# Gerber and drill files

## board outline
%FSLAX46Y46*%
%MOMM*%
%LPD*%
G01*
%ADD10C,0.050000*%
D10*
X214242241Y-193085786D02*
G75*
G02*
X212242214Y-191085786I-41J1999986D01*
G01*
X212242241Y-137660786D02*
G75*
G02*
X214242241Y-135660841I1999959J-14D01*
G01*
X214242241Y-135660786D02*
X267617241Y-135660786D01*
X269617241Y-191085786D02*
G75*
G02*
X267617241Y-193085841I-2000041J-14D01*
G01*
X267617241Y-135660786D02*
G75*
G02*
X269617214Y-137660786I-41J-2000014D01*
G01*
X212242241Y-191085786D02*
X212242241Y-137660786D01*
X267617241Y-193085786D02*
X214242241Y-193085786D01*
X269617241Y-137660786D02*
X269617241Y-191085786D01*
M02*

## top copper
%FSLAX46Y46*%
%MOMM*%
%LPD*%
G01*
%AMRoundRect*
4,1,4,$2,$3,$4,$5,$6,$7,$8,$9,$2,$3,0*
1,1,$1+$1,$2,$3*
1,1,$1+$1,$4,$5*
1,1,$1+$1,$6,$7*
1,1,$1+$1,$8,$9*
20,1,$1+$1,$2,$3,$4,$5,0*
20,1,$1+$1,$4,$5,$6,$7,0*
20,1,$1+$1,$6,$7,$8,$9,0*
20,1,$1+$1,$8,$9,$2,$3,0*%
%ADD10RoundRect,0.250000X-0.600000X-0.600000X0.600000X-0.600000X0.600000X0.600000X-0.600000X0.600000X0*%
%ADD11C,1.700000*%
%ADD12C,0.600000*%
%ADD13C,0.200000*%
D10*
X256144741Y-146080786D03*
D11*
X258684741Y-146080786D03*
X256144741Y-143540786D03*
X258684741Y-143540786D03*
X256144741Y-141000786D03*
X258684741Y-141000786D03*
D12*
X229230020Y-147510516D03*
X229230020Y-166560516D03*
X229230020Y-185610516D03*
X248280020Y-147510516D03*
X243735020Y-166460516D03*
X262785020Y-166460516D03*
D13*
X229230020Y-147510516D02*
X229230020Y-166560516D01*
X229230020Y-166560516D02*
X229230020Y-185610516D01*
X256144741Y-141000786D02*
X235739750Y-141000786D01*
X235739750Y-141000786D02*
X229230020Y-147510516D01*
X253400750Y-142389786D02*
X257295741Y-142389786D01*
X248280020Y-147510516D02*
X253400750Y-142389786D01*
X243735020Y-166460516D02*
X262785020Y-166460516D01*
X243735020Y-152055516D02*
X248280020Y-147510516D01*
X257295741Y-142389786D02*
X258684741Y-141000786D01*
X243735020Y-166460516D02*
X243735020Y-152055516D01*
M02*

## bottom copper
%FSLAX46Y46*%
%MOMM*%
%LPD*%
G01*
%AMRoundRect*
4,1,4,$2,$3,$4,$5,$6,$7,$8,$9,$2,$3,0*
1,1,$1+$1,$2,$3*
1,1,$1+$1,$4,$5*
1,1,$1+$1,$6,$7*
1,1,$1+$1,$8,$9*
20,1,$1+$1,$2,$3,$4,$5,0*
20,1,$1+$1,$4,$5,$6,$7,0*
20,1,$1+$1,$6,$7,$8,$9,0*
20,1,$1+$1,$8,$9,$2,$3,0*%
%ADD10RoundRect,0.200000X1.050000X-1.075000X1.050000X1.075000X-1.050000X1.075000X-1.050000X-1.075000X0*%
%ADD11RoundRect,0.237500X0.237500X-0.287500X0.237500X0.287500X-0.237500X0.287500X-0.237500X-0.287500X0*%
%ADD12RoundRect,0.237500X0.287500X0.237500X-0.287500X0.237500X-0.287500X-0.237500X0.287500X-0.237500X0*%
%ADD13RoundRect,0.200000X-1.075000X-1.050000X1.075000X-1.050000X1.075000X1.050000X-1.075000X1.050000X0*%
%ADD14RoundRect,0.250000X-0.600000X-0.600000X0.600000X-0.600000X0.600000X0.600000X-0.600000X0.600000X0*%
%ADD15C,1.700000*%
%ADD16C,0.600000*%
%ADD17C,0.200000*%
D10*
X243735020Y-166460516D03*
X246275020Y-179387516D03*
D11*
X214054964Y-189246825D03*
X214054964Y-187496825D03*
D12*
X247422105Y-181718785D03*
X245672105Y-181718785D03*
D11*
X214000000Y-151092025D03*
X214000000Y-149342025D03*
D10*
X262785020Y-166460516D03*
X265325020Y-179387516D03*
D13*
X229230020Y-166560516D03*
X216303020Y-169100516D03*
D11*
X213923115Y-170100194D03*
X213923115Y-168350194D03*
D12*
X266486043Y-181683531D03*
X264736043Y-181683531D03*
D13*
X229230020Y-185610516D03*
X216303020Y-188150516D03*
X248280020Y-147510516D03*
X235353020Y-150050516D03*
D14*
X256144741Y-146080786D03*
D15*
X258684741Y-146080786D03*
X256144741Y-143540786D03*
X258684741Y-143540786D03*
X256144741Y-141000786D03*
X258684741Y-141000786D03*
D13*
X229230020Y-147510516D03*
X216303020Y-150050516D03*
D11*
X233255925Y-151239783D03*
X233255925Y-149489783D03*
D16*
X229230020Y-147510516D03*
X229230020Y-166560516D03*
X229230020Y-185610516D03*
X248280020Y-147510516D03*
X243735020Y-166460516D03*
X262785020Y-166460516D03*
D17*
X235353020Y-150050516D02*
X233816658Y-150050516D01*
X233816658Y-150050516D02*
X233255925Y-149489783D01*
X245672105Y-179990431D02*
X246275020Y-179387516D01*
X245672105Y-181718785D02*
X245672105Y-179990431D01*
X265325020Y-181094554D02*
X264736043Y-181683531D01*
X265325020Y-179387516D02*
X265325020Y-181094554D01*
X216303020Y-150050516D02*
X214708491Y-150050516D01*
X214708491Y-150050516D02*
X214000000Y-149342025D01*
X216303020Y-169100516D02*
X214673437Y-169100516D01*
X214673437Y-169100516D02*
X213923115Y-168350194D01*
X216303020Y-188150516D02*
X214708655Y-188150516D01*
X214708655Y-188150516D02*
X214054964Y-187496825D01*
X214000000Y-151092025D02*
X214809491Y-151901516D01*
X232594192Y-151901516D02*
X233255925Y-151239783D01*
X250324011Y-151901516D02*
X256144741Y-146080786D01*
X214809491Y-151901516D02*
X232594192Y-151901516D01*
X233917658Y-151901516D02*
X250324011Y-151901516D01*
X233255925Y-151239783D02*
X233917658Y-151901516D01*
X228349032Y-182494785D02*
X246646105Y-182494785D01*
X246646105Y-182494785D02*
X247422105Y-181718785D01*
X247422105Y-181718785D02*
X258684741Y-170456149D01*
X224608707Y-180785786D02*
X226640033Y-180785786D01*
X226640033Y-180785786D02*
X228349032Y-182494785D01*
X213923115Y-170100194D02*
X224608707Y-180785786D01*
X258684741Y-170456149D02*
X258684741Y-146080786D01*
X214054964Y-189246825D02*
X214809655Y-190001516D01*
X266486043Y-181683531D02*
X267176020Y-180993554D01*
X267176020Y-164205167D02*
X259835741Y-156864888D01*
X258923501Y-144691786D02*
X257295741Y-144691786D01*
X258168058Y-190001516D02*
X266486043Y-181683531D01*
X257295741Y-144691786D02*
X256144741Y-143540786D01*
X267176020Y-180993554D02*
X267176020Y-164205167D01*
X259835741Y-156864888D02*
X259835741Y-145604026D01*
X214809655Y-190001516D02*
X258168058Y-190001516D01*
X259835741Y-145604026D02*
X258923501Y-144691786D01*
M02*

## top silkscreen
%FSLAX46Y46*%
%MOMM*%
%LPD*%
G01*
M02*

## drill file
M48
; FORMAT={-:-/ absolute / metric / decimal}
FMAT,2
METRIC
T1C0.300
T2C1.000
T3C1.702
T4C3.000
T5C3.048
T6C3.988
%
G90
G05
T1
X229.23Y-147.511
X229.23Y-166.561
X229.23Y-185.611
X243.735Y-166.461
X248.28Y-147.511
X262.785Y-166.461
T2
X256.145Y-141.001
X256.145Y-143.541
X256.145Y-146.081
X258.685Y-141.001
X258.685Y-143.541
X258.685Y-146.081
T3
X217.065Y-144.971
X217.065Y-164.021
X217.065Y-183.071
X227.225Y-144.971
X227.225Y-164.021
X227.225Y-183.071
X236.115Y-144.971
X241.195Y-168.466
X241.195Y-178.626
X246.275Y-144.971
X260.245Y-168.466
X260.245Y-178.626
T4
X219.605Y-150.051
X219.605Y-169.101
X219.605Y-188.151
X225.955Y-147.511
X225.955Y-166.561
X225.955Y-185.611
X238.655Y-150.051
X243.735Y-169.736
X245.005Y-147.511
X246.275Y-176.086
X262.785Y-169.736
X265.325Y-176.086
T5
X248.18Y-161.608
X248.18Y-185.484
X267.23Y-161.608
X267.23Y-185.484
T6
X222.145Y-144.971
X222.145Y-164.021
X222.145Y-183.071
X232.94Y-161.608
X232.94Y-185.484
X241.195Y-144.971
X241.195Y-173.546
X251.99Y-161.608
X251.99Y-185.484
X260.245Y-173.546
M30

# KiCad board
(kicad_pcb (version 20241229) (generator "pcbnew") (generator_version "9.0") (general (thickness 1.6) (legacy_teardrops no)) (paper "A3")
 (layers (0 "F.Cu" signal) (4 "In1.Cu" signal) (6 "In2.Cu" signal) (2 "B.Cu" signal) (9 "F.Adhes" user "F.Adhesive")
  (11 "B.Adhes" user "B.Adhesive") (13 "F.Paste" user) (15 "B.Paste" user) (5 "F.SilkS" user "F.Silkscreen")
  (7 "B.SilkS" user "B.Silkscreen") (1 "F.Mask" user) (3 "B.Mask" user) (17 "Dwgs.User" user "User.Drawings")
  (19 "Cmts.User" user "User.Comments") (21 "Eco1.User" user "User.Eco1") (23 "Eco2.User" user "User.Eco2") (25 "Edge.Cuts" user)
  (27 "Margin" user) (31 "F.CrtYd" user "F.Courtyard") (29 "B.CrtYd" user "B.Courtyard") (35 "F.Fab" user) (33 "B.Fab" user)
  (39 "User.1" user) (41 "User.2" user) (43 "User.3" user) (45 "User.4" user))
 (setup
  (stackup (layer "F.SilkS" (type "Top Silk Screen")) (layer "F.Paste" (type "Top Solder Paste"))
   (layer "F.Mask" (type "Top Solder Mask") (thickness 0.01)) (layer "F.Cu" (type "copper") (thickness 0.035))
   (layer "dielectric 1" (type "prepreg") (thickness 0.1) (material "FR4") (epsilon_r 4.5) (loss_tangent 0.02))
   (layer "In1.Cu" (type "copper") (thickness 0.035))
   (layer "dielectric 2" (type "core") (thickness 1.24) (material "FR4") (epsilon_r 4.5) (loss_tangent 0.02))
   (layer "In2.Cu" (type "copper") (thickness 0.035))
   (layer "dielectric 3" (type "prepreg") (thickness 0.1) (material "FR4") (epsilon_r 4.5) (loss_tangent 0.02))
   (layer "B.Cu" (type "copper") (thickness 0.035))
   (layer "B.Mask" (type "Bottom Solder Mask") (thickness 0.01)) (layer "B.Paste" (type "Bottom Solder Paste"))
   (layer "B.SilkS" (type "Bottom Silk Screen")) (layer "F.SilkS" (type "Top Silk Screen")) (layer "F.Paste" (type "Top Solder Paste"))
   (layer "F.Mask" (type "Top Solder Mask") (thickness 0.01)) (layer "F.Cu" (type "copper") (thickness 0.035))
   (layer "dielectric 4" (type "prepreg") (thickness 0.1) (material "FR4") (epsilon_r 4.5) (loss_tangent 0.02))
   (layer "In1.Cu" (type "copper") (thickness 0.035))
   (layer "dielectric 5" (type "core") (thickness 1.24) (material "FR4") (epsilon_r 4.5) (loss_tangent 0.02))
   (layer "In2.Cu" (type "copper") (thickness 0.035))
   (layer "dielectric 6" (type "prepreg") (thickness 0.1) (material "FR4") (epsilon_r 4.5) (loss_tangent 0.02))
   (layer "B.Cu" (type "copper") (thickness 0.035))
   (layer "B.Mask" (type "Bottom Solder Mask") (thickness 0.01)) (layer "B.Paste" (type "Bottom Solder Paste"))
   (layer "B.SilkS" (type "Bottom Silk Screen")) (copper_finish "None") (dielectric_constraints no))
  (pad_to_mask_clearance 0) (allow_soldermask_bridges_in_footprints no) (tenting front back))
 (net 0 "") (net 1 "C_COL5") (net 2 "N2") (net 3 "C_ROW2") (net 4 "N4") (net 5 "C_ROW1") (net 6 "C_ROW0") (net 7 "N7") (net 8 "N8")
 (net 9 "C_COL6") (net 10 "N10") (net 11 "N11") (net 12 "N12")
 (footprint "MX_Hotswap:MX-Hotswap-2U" (layer "B.Cu") (at 241.19502 173.545516 90)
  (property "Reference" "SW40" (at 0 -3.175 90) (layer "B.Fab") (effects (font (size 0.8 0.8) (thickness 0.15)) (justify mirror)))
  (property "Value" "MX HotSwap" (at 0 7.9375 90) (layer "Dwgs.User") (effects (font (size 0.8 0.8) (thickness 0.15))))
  (pad "" np_thru_hole circle (at -11.938 -8.255 90) (size 3.9878 3.9878) (drill 3.9878) (layers "*.Cu" "*.Mask"))
  (pad "" np_thru_hole circle (at -11.938 6.985 90) (size 3.048 3.048) (drill 3.048) (layers "*.Cu" "*.Mask"))
  (pad "" np_thru_hole circle (at -5.08 0 138.099) (size 1.7018 1.7018) (drill 1.7018) (layers "*.Cu" "*.Mask"))
  (pad "" np_thru_hole circle (at -2.54 5.08 90) (size 3 3) (drill 3) (layers "*.Cu" "*.Mask"))
  (pad "" np_thru_hole circle (at 0 0 90) (size 3.9878 3.9878) (drill 3.9878) (layers "*.Cu" "*.Mask"))
  (pad "" np_thru_hole circle (at 3.81 2.540001 90) (size 3 3) (drill 3) (layers "*.Cu" "*.Mask"))
  (pad "" np_thru_hole circle (at 5.08 0 138.099) (size 1.7018 1.7018) (drill 1.7018) (layers "*.Cu" "*.Mask"))
  (pad "" np_thru_hole circle (at 11.938 -8.255 90) (size 3.9878 3.9878) (drill 3.9878) (layers "*.Cu" "*.Mask"))
  (pad "" np_thru_hole circle (at 11.938 6.984999 90) (size 3.048 3.048) (drill 3.048) (layers "*.Cu" "*.Mask"))
  (pad "1" smd roundrect (at 7.085 2.54 90) (size 2.55 2.5) (layers "B.Cu" "B.Mask" "B.Paste") (roundrect_rratio 0.08) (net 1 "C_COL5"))
  (pad "2" smd roundrect (at -5.842 5.08 90) (size 2.55 2.5) (layers "B.Cu" "B.Mask" "B.Paste") (roundrect_rratio 0.08) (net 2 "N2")))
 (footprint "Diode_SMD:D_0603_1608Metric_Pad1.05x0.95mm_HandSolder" (layer "B.Cu") (at 214.054964 188.371825 90)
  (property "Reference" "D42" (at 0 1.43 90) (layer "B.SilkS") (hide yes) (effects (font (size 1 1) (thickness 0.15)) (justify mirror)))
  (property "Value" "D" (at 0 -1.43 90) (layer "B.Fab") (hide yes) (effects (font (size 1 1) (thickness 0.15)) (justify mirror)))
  (pad "1" smd roundrect (at -0.875 0 90) (size 1.05 0.95) (layers "B.Cu" "B.Mask" "B.Paste") (roundrect_rratio 0.25) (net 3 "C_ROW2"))
  (pad "2" smd roundrect (at 0.875 0 90) (size 1.05 0.95) (layers "B.Cu" "B.Mask" "B.Paste") (roundrect_rratio 0.25) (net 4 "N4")))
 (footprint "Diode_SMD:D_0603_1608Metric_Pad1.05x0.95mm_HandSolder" (layer "B.Cu") (at 246.547105 181.718785 180)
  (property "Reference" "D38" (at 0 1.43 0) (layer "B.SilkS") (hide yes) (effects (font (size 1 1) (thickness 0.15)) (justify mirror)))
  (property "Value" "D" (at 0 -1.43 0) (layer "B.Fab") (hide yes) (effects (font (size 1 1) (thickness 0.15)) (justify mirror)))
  (pad "1" smd roundrect (at -0.875 0 180) (size 1.05 0.95) (layers "B.Cu" "B.Mask" "B.Paste") (roundrect_rratio 0.25) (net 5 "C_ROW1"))
  (pad "2" smd roundrect (at 0.875 0 180) (size 1.05 0.95) (layers "B.Cu" "B.Mask" "B.Paste") (roundrect_rratio 0.25) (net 2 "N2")))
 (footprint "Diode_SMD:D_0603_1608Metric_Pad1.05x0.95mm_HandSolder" (layer "B.Cu") (at 214 150.217025 90)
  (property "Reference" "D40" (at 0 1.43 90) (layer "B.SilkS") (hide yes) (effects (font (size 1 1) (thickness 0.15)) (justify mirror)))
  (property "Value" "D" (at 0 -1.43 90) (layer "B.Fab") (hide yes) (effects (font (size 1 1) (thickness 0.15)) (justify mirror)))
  (pad "1" smd roundrect (at -0.875 0 90) (size 1.05 0.95) (layers "B.Cu" "B.Mask" "B.Paste") (roundrect_rratio 0.25) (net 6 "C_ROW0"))
  (pad "2" smd roundrect (at 0.875 0 90) (size 1.05 0.95) (layers "B.Cu" "B.Mask" "B.Paste") (roundrect_rratio 0.25) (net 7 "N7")))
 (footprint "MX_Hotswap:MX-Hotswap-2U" (layer "B.Cu") (at 260.24502 173.545516 90)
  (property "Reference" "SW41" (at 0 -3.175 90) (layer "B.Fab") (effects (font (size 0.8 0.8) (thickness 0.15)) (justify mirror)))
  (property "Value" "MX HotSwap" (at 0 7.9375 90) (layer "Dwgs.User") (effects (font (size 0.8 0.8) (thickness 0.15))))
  (pad "" np_thru_hole circle (at -11.938 -8.255 90) (size 3.9878 3.9878) (drill 3.9878) (layers "*.Cu" "*.Mask"))
  (pad "" np_thru_hole circle (at -11.938 6.985 90) (size 3.048 3.048) (drill 3.048) (layers "*.Cu" "*.Mask"))
  (pad "" np_thru_hole circle (at -5.08 0 138.099) (size 1.7018 1.7018) (drill 1.7018) (layers "*.Cu" "*.Mask"))
  (pad "" np_thru_hole circle (at -2.54 5.08 90) (size 3 3) (drill 3) (layers "*.Cu" "*.Mask"))
  (pad "" np_thru_hole circle (at 0 0 90) (size 3.9878 3.9878) (drill 3.9878) (layers "*.Cu" "*.Mask"))
  (pad "" np_thru_hole circle (at 3.81 2.540001 90) (size 3 3) (drill 3) (layers "*.Cu" "*.Mask"))
  (pad "" np_thru_hole circle (at 5.08 0 138.099) (size 1.7018 1.7018) (drill 1.7018) (layers "*.Cu" "*.Mask"))
  (pad "" np_thru_hole circle (at 11.938 -8.255 90) (size 3.9878 3.9878) (drill 3.9878) (layers "*.Cu" "*.Mask"))
  (pad "" np_thru_hole circle (at 11.938 6.984999 90) (size 3.048 3.048) (drill 3.048) (layers "*.Cu" "*.Mask"))
  (pad "1" smd roundrect (at 7.085 2.54 90) (size 2.55 2.5) (layers "B.Cu" "B.Mask" "B.Paste") (roundrect_rratio 0.08) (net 1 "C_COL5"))
  (pad "2" smd roundrect (at -5.842 5.08 90) (size 2.55 2.5) (layers "B.Cu" "B.Mask" "B.Paste") (roundrect_rratio 0.08) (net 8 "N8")))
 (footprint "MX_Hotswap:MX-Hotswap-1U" (layer "B.Cu") (at 222.14502 164.020516)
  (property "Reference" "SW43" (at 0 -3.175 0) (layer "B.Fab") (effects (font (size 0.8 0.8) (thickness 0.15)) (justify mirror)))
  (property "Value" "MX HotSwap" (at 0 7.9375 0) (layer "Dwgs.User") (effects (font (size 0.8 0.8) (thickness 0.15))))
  (pad "" np_thru_hole circle (at -5.08 0 48.099) (size 1.7018 1.7018) (drill 1.7018) (layers "*.Cu" "*.Mask"))
  (pad "" np_thru_hole circle (at -2.54 5.08) (size 3 3) (drill 3) (layers "*.Cu" "*.Mask"))
  (pad "" np_thru_hole circle (at 0 0) (size 3.9878 3.9878) (drill 3.9878) (layers "*.Cu" "*.Mask"))
  (pad "" np_thru_hole circle (at 3.81 2.540001) (size 3 3) (drill 3) (layers "*.Cu" "*.Mask"))
  (pad "" np_thru_hole circle (at 5.08 0 48.099) (size 1.7018 1.7018) (drill 1.7018) (layers "*.Cu" "*.Mask"))
  (pad "1" smd roundrect (at 7.085 2.54) (size 2.55 2.5) (layers "B.Cu" "B.Mask" "B.Paste") (roundrect_rratio 0.08) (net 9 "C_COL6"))
  (pad "2" smd roundrect (at -5.842 5.08) (size 2.55 2.5) (layers "B.Cu" "B.Mask" "B.Paste") (roundrect_rratio 0.08) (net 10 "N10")))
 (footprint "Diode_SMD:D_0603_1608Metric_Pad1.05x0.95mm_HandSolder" (layer "B.Cu") (at 213.923115 169.225194 90)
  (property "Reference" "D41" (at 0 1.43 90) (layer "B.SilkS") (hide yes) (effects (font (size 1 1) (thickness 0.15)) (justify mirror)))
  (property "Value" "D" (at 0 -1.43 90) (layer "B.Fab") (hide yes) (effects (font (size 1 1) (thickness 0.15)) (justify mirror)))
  (pad "1" smd roundrect (at -0.875 0 90) (size 1.05 0.95) (layers "B.Cu" "B.Mask" "B.Paste") (roundrect_rratio 0.25) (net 5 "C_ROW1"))
  (pad "2" smd roundrect (at 0.875 0 90) (size 1.05 0.95) (layers "B.Cu" "B.Mask" "B.Paste") (roundrect_rratio 0.25) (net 10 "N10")))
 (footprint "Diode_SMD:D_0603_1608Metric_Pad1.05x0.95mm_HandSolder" (layer "B.Cu") (at 265.611043 181.683531 180)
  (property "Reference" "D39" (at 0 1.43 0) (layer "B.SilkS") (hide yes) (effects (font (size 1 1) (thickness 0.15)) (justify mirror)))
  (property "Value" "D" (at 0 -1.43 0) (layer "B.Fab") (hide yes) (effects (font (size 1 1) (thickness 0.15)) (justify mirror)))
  (pad "1" smd roundrect (at -0.875 0 180) (size 1.05 0.95) (layers "B.Cu" "B.Mask" "B.Paste") (roundrect_rratio 0.25) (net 3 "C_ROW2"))
  (pad "2" smd roundrect (at 0.875 0 180) (size 1.05 0.95) (layers "B.Cu" "B.Mask" "B.Paste") (roundrect_rratio 0.25) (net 8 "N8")))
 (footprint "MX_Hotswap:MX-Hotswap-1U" (layer "B.Cu") (at 222.14502 183.070516)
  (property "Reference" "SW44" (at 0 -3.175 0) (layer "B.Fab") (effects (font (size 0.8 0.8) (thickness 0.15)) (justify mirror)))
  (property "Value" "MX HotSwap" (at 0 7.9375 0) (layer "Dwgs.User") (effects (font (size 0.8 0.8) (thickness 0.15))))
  (pad "" np_thru_hole circle (at -5.08 0 48.099) (size 1.7018 1.7018) (drill 1.7018) (layers "*.Cu" "*.Mask"))
  (pad "" np_thru_hole circle (at -2.54 5.08) (size 3 3) (drill 3) (layers "*.Cu" "*.Mask"))
  (pad "" np_thru_hole circle (at 0 0) (size 3.9878 3.9878) (drill 3.9878) (layers "*.Cu" "*.Mask"))
  (pad "" np_thru_hole circle (at 3.81 2.540001) (size 3 3) (drill 3) (layers "*.Cu" "*.Mask"))
  (pad "" np_thru_hole circle (at 5.08 0 48.099) (size 1.7018 1.7018) (drill 1.7018) (layers "*.Cu" "*.Mask"))
  (pad "1" smd roundrect (at 7.085 2.54) (size 2.55 2.5) (layers "B.Cu" "B.Mask" "B.Paste") (roundrect_rratio 0.08) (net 9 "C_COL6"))
  (pad "2" smd roundrect (at -5.842 5.08) (size 2.55 2.5) (layers "B.Cu" "B.Mask" "B.Paste") (roundrect_rratio 0.08) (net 4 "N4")))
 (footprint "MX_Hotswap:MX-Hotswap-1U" (layer "B.Cu") (at 241.19502 144.970516)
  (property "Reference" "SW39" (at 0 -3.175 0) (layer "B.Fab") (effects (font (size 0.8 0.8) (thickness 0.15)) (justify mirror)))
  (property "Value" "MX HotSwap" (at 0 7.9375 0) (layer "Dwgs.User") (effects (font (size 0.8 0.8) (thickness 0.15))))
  (pad "" np_thru_hole circle (at -5.08 0 48.099) (size 1.7018 1.7018) (drill 1.7018) (layers "*.Cu" "*.Mask"))
  (pad "" np_thru_hole circle (at -2.54 5.08) (size 3 3) (drill 3) (layers "*.Cu" "*.Mask"))
  (pad "" np_thru_hole circle (at 0 0) (size 3.9878 3.9878) (drill 3.9878) (layers "*.Cu" "*.Mask"))
  (pad "" np_thru_hole circle (at 3.81 2.540001) (size 3 3) (drill 3) (layers "*.Cu" "*.Mask"))
  (pad "" np_thru_hole circle (at 5.08 0 48.099) (size 1.7018 1.7018) (drill 1.7018) (layers "*.Cu" "*.Mask"))
  (pad "1" smd roundrect (at 7.085 2.54) (size 2.55 2.5) (layers "B.Cu" "B.Mask" "B.Paste") (roundrect_rratio 0.08) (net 1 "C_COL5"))
  (pad "2" smd roundrect (at -5.842 5.08) (size 2.55 2.5) (layers "B.Cu" "B.Mask" "B.Paste") (roundrect_rratio 0.08) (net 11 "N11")))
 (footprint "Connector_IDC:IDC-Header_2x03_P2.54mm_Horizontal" (layer "B.Cu") (at 256.144741 146.080786)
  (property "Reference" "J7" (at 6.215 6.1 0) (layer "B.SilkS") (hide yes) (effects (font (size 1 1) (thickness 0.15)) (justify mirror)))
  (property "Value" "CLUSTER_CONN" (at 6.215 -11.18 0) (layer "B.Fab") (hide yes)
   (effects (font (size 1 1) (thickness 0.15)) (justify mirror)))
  (pad "1" thru_hole roundrect (at 0 0) (size 1.7 1.7) (drill 1) (layers "*.Cu" "*.Mask") (remove_unused_layers no)
   (roundrect_rratio 0.147059) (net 6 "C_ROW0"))
  (pad "2" thru_hole circle (at 2.54 0) (size 1.7 1.7) (drill 1) (layers "*.Cu" "*.Mask") (remove_unused_layers no) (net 5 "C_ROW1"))
  (pad "3" thru_hole circle (at 0 -2.54) (size 1.7 1.7) (drill 1) (layers "*.Cu" "*.Mask") (remove_unused_layers no) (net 3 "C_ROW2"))
  (pad "4" thru_hole circle (at 2.54 -2.54) (size 1.7 1.7) (drill 1) (layers "*.Cu" "*.Mask") (remove_unused_layers no) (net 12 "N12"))
  (pad "5" thru_hole circle (at 0 -5.08) (size 1.7 1.7) (drill 1) (layers "*.Cu" "*.Mask") (remove_unused_layers no) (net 9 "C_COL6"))
  (pad "6" thru_hole circle (at 2.54 -5.08) (size 1.7 1.7) (drill 1) (layers "*.Cu" "*.Mask") (remove_unused_layers no) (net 1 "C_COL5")))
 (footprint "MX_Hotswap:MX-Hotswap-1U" (layer "B.Cu") (at 222.14502 144.970516)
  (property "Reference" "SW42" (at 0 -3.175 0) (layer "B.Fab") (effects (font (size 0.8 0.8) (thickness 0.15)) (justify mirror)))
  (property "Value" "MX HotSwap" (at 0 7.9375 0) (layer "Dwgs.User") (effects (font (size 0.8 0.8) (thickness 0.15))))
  (pad "" np_thru_hole circle (at -5.08 0 48.099) (size 1.7018 1.7018) (drill 1.7018) (layers "*.Cu" "*.Mask"))
  (pad "" np_thru_hole circle (at -2.54 5.08) (size 3 3) (drill 3) (layers "*.Cu" "*.Mask"))
  (pad "" np_thru_hole circle (at 0 0) (size 3.9878 3.9878) (drill 3.9878) (layers "*.Cu" "*.Mask"))
  (pad "" np_thru_hole circle (at 3.81 2.540001) (size 3 3) (drill 3) (layers "*.Cu" "*.Mask"))
  (pad "" np_thru_hole circle (at 5.08 0 48.099) (size 1.7018 1.7018) (drill 1.7018) (layers "*.Cu" "*.Mask"))
  (pad "1" smd roundrect (at 7.085 2.54) (size 2.55 2.5) (layers "B.Cu" "B.Mask" "B.Paste") (roundrect_rratio 0.08) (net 9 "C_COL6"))
  (pad "2" smd roundrect (at -5.842 5.08) (size 2.55 2.5) (layers "B.Cu" "B.Mask" "B.Paste") (roundrect_rratio 0.08) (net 7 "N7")))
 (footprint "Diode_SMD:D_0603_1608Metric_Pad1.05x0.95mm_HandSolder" (layer "B.Cu") (at 233.255925 150.364783 90)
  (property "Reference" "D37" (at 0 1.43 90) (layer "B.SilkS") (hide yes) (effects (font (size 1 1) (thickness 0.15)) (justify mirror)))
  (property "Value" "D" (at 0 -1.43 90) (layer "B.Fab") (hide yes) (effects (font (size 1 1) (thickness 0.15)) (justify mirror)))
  (pad "1" smd roundrect (at -0.875 0 90) (size 1.05 0.95) (layers "B.Cu" "B.Mask" "B.Paste") (roundrect_rratio 0.25) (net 6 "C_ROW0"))
  (pad "2" smd roundrect (at 0.875 0 90) (size 1.05 0.95) (layers "B.Cu" "B.Mask" "B.Paste") (roundrect_rratio 0.25) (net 11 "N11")))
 (gr_arc (start 214.242241 193.085786) (mid 212.828027 192.5) (end 212.242241 191.085786) (stroke (width 0.05) (type default))
  (layer "Edge.Cuts"))
 (gr_arc (start 212.242241 137.660786) (mid 212.828027 136.246572) (end 214.242241 135.660786) (stroke (width 0.05) (type default))
  (layer "Edge.Cuts"))
 (gr_line (start 214.242241 135.660786) (end 267.617241 135.660786) (stroke (width 0.05) (type default)) (layer "Edge.Cuts"))
 (gr_arc (start 269.617241 191.085786) (mid 269.031455 192.5) (end 267.617241 193.085786) (stroke (width 0.05) (type default))
  (layer "Edge.Cuts"))
 (gr_arc (start 267.617241 135.660786) (mid 269.031455 136.246572) (end 269.617241 137.660786) (stroke (width 0.05) (type default))
  (layer "Edge.Cuts"))
 (gr_line (start 212.242241 191.085786) (end 212.242241 137.660786) (stroke (width 0.05) (type default)) (layer "Edge.Cuts"))
 (gr_line (start 267.617241 193.085786) (end 214.242241 193.085786) (stroke (width 0.05) (type default)) (layer "Edge.Cuts"))
 (gr_line (start 269.617241 137.660786) (end 269.617241 191.085786) (stroke (width 0.05) (type default)) (layer "Edge.Cuts"))
 (segment (start 235.35302 150.050516) (end 233.816658 150.050516) (width 0.2) (layer "B.Cu") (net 11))
 (segment (start 233.816658 150.050516) (end 233.255925 149.489783) (width 0.2) (layer "B.Cu") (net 11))
 (segment (start 245.672105 179.990431) (end 246.27502 179.387516) (width 0.2) (layer "B.Cu") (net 2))
 (segment (start 245.672105 181.718785) (end 245.672105 179.990431) (width 0.2) (layer "B.Cu") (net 2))
 (segment (start 265.32502 181.094554) (end 264.736043 181.683531) (width 0.2) (layer "B.Cu") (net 8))
 (segment (start 265.32502 179.387516) (end 265.32502 181.094554) (width 0.2) (layer "B.Cu") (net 8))
 (segment (start 216.30302 150.050516) (end 214.708491 150.050516) (width 0.2) (layer "B.Cu") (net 7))
 (segment (start 214.708491 150.050516) (end 214 149.342025) (width 0.2) (layer "B.Cu") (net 7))
 (segment (start 216.30302 169.100516) (end 214.673437 169.100516) (width 0.2) (layer "B.Cu") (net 10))
 (segment (start 214.673437 169.100516) (end 213.923115 168.350194) (width 0.2) (layer "B.Cu") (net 10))
 (segment (start 216.30302 188.150516) (end 214.708655 188.150516) (width 0.2) (layer "B.Cu") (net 4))
 (segment (start 214.708655 188.150516) (end 214.054964 187.496825) (width 0.2) (layer "B.Cu") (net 4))
 (segment (start 214 151.092025) (end 214.809491 151.901516) (width 0.2) (layer "B.Cu") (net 6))
 (segment (start 232.594192 151.901516) (end 233.255925 151.239783) (width 0.2) (layer "B.Cu") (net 6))
 (segment (start 250.324011 151.901516) (end 256.144741 146.080786) (width 0.2) (layer "B.Cu") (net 6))
 (segment (start 214.809491 151.901516) (end 232.594192 151.901516) (width 0.2) (layer "B.Cu") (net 6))
 (segment (start 233.917658 151.901516) (end 250.324011 151.901516) (width 0.2) (layer "B.Cu") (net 6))
 (segment (start 233.255925 151.239783) (end 233.917658 151.901516) (width 0.2) (layer "B.Cu") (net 6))
 (segment (start 228.349032 182.494785) (end 246.646105 182.494785) (width 0.2) (layer "B.Cu") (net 5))
 (segment (start 246.646105 182.494785) (end 247.422105 181.718785) (width 0.2) (layer "B.Cu") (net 5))
 (segment (start 247.422105 181.718785) (end 258.684741 170.456149) (width 0.2) (layer "B.Cu") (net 5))
 (segment (start 224.608707 180.785786) (end 226.640033 180.785786) (width 0.2) (layer "B.Cu") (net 5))
 (segment (start 226.640033 180.785786) (end 228.349032 182.494785) (width 0.2) (layer "B.Cu") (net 5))
 (segment (start 213.923115 170.100194) (end 224.608707 180.785786) (width 0.2) (layer "B.Cu") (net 5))
 (segment (start 258.684741 170.456149) (end 258.684741 146.080786) (width 0.2) (layer "B.Cu") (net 5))
 (segment (start 214.054964 189.246825) (end 214.809655 190.001516) (width 0.2) (layer "B.Cu") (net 3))
 (segment (start 266.486043 181.683531) (end 267.17602 180.993554) (width 0.2) (layer "B.Cu") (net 3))
 (segment (start 267.17602 164.205167) (end 259.835741 156.864888) (width 0.2) (layer "B.Cu") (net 3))
 (segment (start 258.923501 144.691786) (end 257.295741 144.691786) (width 0.2) (layer "B.Cu") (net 3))
 (segment (start 258.168058 190.001516) (end 266.486043 181.683531) (width 0.2) (layer "B.Cu") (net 3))
 (segment (start 257.295741 144.691786) (end 256.144741 143.540786) (width 0.2) (layer "B.Cu") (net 3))
 (segment (start 267.17602 180.993554) (end 267.17602 164.205167) (width 0.2) (layer "B.Cu") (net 3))
 (segment (start 259.835741 156.864888) (end 259.835741 145.604026) (width 0.2) (layer "B.Cu") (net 3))
 (segment (start 214.809655 190.001516) (end 258.168058 190.001516) (width 0.2) (layer "B.Cu") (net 3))
 (segment (start 259.835741 145.604026) (end 258.923501 144.691786) (width 0.2) (layer "B.Cu") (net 3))
 (segment (start 229.23002 147.510516) (end 229.23002 166.560516) (width 0.2) (layer "F.Cu") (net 9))
 (segment (start 229.23002 166.560516) (end 229.23002 185.610516) (width 0.2) (layer "F.Cu") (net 9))
 (segment (start 256.144741 141.000786) (end 235.73975 141.000786) (width 0.2) (layer "F.Cu") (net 9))
 (segment (start 235.73975 141.000786) (end 229.23002 147.510516) (width 0.2) (layer "F.Cu") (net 9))
 (via (at 229.23002 147.510516) (size 0.6) (drill 0.3) (layers "F.Cu" "B.Cu") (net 9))
 (via (at 229.23002 166.560516) (size 0.6) (drill 0.3) (layers "F.Cu" "B.Cu") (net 9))
 (via (at 229.23002 185.610516) (size 0.6) (drill 0.3) (layers "F.Cu" "B.Cu") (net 9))
 (segment (start 253.40075 142.389786) (end 257.295741 142.389786) (width 0.2) (layer "F.Cu") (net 1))
 (segment (start 248.28002 147.510516) (end 253.40075 142.389786) (width 0.2) (layer "F.Cu") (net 1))
 (segment (start 243.73502 166.460516) (end 262.78502 166.460516) (width 0.2) (layer "F.Cu") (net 1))
 (segment (start 243.73502 152.055516) (end 248.28002 147.510516) (width 0.2) (layer "F.Cu") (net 1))
 (segment (start 257.295741 142.389786) (end 258.684741 141.000786) (width 0.2) (layer "F.Cu") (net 1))
 (segment (start 243.73502 166.460516) (end 243.73502 152.055516) (width 0.2) (layer "F.Cu") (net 1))
 (via (at 248.28002 147.510516) (size 0.6) (drill 0.3) (layers "F.Cu" "B.Cu") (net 1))
 (via (at 243.73502 166.460516) (size 0.6) (drill 0.3) (layers "F.Cu" "B.Cu") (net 1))
 (via (at 262.78502 166.460516) (size 0.6) (drill 0.3) (layers "F.Cu" "B.Cu") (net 1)))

